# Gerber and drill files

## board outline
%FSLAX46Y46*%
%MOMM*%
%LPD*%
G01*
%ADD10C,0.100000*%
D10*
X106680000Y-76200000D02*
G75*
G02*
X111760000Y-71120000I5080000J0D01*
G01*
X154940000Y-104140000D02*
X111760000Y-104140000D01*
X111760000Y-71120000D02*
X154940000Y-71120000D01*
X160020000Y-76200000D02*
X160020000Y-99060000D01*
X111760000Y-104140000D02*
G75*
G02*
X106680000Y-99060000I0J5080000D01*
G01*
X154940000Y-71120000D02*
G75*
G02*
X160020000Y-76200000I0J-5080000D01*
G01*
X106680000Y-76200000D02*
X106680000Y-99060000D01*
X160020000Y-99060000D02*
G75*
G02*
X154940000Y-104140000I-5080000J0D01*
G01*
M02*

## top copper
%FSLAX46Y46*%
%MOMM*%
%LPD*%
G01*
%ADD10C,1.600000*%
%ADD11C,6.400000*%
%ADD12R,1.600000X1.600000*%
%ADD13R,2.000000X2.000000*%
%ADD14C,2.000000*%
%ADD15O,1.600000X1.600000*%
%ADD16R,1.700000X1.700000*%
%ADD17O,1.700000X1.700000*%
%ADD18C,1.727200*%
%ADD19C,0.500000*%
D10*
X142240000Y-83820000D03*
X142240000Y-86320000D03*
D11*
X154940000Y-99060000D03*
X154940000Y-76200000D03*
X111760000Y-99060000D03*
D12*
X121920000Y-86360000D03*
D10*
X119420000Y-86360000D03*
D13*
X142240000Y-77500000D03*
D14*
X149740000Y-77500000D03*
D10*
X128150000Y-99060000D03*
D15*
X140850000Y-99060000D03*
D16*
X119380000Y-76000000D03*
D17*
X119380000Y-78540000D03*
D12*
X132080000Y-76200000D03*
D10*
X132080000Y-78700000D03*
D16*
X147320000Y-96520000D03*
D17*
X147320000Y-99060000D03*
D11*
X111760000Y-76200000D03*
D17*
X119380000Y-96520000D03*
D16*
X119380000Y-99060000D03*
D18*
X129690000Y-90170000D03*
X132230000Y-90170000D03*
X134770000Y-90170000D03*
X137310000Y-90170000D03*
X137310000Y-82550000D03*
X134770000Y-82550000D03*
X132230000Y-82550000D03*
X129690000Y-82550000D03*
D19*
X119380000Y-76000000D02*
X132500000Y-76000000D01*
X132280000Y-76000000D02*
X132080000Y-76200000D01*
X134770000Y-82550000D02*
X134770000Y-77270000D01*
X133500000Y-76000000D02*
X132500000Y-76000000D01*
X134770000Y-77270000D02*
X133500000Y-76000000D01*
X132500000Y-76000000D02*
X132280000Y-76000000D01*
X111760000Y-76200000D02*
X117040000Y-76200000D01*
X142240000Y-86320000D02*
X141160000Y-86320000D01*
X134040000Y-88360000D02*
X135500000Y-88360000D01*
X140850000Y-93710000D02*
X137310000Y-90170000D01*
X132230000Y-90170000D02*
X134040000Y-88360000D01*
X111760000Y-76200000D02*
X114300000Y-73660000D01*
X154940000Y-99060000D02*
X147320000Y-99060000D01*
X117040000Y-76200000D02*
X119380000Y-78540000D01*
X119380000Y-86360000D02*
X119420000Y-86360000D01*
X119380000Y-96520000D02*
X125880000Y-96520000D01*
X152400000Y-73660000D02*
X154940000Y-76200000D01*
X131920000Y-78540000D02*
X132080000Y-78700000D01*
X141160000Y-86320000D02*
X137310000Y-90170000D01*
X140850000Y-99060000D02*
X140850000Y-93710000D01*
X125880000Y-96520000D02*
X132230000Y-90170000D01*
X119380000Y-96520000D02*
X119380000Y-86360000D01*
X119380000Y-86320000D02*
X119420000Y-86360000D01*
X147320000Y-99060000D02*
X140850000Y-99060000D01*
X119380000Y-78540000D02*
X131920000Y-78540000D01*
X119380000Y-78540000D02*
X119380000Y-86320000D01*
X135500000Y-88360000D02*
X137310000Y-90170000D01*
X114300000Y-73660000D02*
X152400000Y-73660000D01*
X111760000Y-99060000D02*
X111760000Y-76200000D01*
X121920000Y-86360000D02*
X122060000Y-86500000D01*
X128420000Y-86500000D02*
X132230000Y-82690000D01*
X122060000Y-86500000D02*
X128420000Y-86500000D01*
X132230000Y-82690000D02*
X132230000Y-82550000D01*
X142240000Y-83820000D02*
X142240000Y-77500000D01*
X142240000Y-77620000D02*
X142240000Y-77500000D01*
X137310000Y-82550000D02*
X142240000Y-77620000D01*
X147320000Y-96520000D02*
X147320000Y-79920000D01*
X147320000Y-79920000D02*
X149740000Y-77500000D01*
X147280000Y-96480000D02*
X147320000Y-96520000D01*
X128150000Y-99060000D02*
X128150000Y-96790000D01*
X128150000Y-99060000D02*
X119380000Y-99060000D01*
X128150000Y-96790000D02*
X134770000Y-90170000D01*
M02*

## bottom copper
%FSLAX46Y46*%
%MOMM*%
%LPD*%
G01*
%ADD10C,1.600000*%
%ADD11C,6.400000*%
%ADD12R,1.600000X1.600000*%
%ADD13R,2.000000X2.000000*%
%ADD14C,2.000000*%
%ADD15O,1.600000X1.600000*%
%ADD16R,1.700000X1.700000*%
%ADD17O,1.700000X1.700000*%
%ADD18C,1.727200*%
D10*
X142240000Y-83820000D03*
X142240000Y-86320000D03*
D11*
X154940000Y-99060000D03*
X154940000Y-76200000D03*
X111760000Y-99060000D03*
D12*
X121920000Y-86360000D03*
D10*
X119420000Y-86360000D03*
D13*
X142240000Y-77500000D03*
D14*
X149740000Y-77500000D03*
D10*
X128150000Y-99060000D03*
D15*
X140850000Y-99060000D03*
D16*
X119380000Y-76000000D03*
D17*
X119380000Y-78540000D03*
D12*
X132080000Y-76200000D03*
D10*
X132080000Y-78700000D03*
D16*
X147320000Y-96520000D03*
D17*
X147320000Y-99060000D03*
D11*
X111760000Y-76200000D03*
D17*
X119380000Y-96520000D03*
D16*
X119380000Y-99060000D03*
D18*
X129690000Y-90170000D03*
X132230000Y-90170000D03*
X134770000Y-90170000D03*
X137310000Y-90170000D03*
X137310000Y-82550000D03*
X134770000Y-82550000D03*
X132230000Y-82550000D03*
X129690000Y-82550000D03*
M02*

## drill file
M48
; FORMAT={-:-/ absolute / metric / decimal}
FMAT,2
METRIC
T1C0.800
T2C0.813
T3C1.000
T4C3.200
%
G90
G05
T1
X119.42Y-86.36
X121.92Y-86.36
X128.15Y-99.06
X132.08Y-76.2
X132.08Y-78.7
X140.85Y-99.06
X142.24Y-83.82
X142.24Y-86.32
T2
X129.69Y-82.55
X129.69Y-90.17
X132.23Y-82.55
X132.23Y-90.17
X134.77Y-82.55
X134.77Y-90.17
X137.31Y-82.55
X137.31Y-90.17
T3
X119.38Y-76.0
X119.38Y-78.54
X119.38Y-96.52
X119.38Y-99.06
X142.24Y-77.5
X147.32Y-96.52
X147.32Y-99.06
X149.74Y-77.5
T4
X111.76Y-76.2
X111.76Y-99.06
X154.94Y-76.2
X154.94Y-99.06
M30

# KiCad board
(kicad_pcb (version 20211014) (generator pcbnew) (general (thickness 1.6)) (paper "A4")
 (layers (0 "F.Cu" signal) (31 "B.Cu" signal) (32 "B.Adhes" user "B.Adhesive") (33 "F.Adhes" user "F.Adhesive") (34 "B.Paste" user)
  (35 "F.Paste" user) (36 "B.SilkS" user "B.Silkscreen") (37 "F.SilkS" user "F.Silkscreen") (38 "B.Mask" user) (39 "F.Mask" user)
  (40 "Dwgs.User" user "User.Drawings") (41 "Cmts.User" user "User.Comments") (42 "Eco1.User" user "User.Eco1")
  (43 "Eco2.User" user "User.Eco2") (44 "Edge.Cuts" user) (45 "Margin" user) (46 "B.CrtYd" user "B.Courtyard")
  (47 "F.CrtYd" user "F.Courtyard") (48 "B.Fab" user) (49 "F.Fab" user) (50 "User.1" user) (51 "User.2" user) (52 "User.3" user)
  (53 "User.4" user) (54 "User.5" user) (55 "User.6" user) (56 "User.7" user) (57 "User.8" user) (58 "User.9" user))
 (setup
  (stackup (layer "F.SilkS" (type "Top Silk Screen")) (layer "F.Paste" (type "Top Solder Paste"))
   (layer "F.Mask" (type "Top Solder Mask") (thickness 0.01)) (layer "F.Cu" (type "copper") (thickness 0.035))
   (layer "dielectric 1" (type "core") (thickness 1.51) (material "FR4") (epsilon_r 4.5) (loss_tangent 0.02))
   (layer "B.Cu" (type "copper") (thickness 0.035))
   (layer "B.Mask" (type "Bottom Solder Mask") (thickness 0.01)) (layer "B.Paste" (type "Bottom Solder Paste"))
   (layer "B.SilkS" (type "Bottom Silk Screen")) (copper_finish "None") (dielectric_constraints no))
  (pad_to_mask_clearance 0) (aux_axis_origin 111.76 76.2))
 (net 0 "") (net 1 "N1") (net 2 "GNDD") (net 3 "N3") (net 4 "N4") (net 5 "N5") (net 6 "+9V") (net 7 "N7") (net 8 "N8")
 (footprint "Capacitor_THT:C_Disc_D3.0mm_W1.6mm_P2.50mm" (layer "F.Cu") (at 142.24 83.82 -90)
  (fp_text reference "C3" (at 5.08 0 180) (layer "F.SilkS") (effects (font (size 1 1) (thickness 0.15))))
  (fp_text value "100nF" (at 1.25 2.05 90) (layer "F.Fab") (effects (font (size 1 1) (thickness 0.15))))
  (pad "1" thru_hole circle (at 0 0 270) (size 1.6 1.6) (drill 0.8) (layers *.Cu *.Mask) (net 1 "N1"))
  (pad "2" thru_hole circle (at 2.5 0 270) (size 1.6 1.6) (drill 0.8) (layers *.Cu *.Mask) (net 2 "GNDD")))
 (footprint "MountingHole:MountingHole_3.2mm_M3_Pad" (layer "F.Cu") (at 154.94 99.06)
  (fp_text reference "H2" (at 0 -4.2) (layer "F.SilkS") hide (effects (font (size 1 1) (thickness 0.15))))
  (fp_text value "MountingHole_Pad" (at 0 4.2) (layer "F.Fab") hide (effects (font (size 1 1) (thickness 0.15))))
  (pad "1" thru_hole circle (at 0 0) (size 6.4 6.4) (drill 3.2) (layers *.Cu *.Mask) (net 2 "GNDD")))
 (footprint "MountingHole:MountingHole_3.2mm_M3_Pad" (layer "F.Cu") (at 154.94 76.2)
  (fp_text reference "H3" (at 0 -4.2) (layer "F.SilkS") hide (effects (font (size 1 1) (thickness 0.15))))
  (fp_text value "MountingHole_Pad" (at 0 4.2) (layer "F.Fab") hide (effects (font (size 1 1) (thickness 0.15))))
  (pad "1" thru_hole circle (at 0 0) (size 6.4 6.4) (drill 3.2) (layers *.Cu *.Mask) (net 2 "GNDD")))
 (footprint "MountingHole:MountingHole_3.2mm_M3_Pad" (layer "F.Cu") (at 111.76 99.06)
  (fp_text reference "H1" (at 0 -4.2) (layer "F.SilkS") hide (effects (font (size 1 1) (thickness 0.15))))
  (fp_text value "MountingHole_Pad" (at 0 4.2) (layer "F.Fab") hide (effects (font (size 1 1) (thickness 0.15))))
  (pad "1" thru_hole circle (at 0 0) (size 6.4 6.4) (drill 3.2) (layers *.Cu *.Mask) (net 2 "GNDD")))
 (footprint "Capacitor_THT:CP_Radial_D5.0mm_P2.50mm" (layer "F.Cu") (at 121.92 86.36 180)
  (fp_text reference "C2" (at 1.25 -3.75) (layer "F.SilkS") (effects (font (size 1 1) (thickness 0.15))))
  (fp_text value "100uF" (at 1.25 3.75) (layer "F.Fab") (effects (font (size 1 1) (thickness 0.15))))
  (pad "1" thru_hole rect (at 0 0 180) (size 1.6 1.6) (drill 0.8) (layers *.Cu *.Mask) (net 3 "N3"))
  (pad "2" thru_hole circle (at 2.5 0 180) (size 1.6 1.6) (drill 0.8) (layers *.Cu *.Mask) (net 2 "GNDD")))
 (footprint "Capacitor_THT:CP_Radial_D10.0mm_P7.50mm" (layer "F.Cu") (at 142.24 77.5)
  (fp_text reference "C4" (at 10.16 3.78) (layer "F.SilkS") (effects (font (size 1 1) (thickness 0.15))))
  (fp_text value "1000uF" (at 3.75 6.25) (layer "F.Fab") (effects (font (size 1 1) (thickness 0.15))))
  (pad "1" thru_hole rect (at 0 0) (size 2 2) (drill 1) (layers *.Cu *.Mask) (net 1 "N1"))
  (pad "2" thru_hole circle (at 7.5 0) (size 2 2) (drill 1) (layers *.Cu *.Mask) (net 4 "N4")))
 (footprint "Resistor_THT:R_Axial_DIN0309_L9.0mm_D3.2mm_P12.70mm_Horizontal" (layer "F.Cu") (at 128.15 99.06)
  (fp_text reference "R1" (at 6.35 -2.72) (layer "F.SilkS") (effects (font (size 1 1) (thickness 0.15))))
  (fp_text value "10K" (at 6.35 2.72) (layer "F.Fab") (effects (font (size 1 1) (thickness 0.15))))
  (pad "1" thru_hole circle (at 0 0) (size 1.6 1.6) (drill 0.8) (layers *.Cu *.Mask) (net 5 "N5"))
  (pad "2" thru_hole oval (at 12.7 0) (size 1.6 1.6) (drill 0.8) (layers *.Cu *.Mask) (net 2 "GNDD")))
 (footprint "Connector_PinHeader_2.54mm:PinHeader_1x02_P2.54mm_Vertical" (layer "F.Cu") (at 119.38 76)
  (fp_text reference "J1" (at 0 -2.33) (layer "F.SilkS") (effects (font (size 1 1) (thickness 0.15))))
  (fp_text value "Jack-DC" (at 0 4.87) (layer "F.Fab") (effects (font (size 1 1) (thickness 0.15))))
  (pad "1" thru_hole rect (at 0 0) (size 1.7 1.7) (drill 1) (layers *.Cu *.Mask) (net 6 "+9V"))
  (pad "2" thru_hole oval (at 0 2.54) (size 1.7 1.7) (drill 1) (layers *.Cu *.Mask) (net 2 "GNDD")))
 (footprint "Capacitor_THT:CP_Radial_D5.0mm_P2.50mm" (layer "F.Cu") (at 132.08 76.2 -90)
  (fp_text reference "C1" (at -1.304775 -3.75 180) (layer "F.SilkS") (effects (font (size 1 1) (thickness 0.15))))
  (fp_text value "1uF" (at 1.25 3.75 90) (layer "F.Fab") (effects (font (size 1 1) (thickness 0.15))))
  (pad "1" thru_hole rect (at 0 0 270) (size 1.6 1.6) (drill 0.8) (layers *.Cu *.Mask) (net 6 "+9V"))
  (pad "2" thru_hole circle (at 2.5 0 270) (size 1.6 1.6) (drill 0.8) (layers *.Cu *.Mask) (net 2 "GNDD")))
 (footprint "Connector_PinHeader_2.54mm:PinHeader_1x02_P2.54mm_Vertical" (layer "F.Cu") (at 147.32 96.52)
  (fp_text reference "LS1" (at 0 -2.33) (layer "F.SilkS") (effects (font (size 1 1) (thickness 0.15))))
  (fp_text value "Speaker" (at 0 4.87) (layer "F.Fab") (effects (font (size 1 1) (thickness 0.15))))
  (pad "1" thru_hole rect (at 0 0) (size 1.7 1.7) (drill 1) (layers *.Cu *.Mask) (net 4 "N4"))
  (pad "2" thru_hole oval (at 0 2.54) (size 1.7 1.7) (drill 1) (layers *.Cu *.Mask) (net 2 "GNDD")))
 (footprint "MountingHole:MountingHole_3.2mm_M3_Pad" (layer "F.Cu") (at 111.76 76.2)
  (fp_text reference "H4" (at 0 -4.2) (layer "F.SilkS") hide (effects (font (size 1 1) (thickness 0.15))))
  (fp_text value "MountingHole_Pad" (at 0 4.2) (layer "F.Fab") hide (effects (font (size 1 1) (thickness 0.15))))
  (pad "1" thru_hole circle (at 0 0) (size 6.4 6.4) (drill 3.2) (layers *.Cu *.Mask) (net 2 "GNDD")))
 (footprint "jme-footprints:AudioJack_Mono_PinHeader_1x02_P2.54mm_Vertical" (layer "F.Cu") (at 119.38 99.06 180)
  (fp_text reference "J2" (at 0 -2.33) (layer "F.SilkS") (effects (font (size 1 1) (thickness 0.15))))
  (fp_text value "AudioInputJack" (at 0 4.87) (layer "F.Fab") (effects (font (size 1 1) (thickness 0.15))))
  (pad "S" thru_hole oval (at 0 2.54 180) (size 1.7 1.7) (drill 1) (layers *.Cu *.Mask) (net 2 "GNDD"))
  (pad "T" thru_hole rect (at 0 0 180) (size 1.7 1.7) (drill 1) (layers *.Cu *.Mask) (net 5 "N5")))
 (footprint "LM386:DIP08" (layer "F.Cu") (at 133.5 86.36)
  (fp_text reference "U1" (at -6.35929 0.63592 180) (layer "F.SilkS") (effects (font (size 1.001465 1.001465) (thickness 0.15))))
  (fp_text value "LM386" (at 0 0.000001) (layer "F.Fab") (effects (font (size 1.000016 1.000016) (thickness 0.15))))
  (pad "1" thru_hole circle locked (at -3.81 3.81) (size 1.7272 1.7272) (drill 0.8128) (layers *.Cu *.Mask) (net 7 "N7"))
  (pad "2" thru_hole circle locked (at -1.27 3.81) (size 1.7272 1.7272) (drill 0.8128) (layers *.Cu *.Mask) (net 2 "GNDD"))
  (pad "3" thru_hole circle locked (at 1.27 3.81) (size 1.7272 1.7272) (drill 0.8128) (layers *.Cu *.Mask) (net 5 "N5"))
  (pad "4" thru_hole circle locked (at 3.81 3.81) (size 1.7272 1.7272) (drill 0.8128) (layers *.Cu *.Mask) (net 2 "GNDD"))
  (pad "5" thru_hole circle locked (at 3.81 -3.81) (size 1.7272 1.7272) (drill 0.8128) (layers *.Cu *.Mask) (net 1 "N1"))
  (pad "6" thru_hole circle locked (at 1.27 -3.81) (size 1.7272 1.7272) (drill 0.8128) (layers *.Cu *.Mask) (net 6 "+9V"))
  (pad "7" thru_hole circle locked (at -1.27 -3.81) (size 1.7272 1.7272) (drill 0.8128) (layers *.Cu *.Mask) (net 3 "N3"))
  (pad "8" thru_hole circle locked (at -3.81 -3.81) (size 1.7272 1.7272) (drill 0.8128) (layers *.Cu *.Mask) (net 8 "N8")))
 (gr_arc (start 106.68 76.2) (mid 108.167898 72.607898) (end 111.76 71.12) (layer "Edge.Cuts") (width 0.1))
 (gr_line (start 154.94 104.14) (end 111.76 104.14) (layer "Edge.Cuts") (width 0.1))
 (gr_line (start 111.76 71.12) (end 154.94 71.12) (layer "Edge.Cuts") (width 0.1))
 (gr_line (start 160.02 76.2) (end 160.02 99.06) (layer "Edge.Cuts") (width 0.1))
 (gr_arc (start 111.76 104.14) (mid 108.167898 102.652102) (end 106.68 99.06) (layer "Edge.Cuts") (width 0.1))
 (gr_arc (start 154.94 71.12) (mid 158.532102 72.607898) (end 160.02 76.2) (layer "Edge.Cuts") (width 0.1))
 (gr_line (start 106.68 76.2) (end 106.68 99.06) (layer "Edge.Cuts") (width 0.1))
 (gr_arc (start 160.02 99.06) (mid 158.532102 102.652102) (end 154.94 104.14) (layer "Edge.Cuts") (width 0.1))
 (segment (start 119.38 76) (end 132.5 76) (width 0.5) (layer "F.Cu") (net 6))
 (segment (start 132.28 76) (end 132.08 76.2) (width 0.5) (layer "F.Cu") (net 6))
 (segment (start 134.77 82.55) (end 134.77 77.27) (width 0.5) (layer "F.Cu") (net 6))
 (segment (start 133.5 76) (end 132.5 76) (width 0.5) (layer "F.Cu") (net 6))
 (segment (start 134.77 77.27) (end 133.5 76) (width 0.5) (layer "F.Cu") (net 6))
 (segment (start 132.5 76) (end 132.28 76) (width 0.5) (layer "F.Cu") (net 6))
 (segment (start 111.76 76.2) (end 117.04 76.2) (width 0.5) (layer "F.Cu") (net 2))
 (segment (start 142.24 86.32) (end 141.16 86.32) (width 0.5) (layer "F.Cu") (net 2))
 (segment (start 134.04 88.36) (end 135.5 88.36) (width 0.5) (layer "F.Cu") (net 2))
 (segment (start 140.85 93.71) (end 137.31 90.17) (width 0.5) (layer "F.Cu") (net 2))
 (segment (start 132.23 90.17) (end 134.04 88.36) (width 0.5) (layer "F.Cu") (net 2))
 (segment (start 111.76 76.2) (end 114.3 73.66) (width 0.5) (layer "F.Cu") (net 2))
 (segment (start 154.94 99.06) (end 147.32 99.06) (width 0.5) (layer "F.Cu") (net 2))
 (segment (start 117.04 76.2) (end 119.38 78.54) (width 0.5) (layer "F.Cu") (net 2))
 (segment (start 119.38 86.36) (end 119.42 86.36) (width 0.5) (layer "F.Cu") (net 2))
 (segment (start 119.38 96.52) (end 125.88 96.52) (width 0.5) (layer "F.Cu") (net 2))
 (segment (start 152.4 73.66) (end 154.94 76.2) (width 0.5) (layer "F.Cu") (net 2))
 (segment (start 131.92 78.54) (end 132.08 78.7) (width 0.5) (layer "F.Cu") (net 2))
 (segment (start 141.16 86.32) (end 137.31 90.17) (width 0.5) (layer "F.Cu") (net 2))
 (segment (start 140.85 99.06) (end 140.85 93.71) (width 0.5) (layer "F.Cu") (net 2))
 (segment (start 125.88 96.52) (end 132.23 90.17) (width 0.5) (layer "F.Cu") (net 2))
 (segment (start 119.38 96.52) (end 119.38 86.36) (width 0.5) (layer "F.Cu") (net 2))
 (segment (start 119.38 86.32) (end 119.42 86.36) (width 0.5) (layer "F.Cu") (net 2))
 (segment (start 147.32 99.06) (end 140.85 99.06) (width 0.5) (layer "F.Cu") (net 2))
 (segment (start 119.38 78.54) (end 131.92 78.54) (width 0.5) (layer "F.Cu") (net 2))
 (segment (start 119.38 78.54) (end 119.38 86.32) (width 0.5) (layer "F.Cu") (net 2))
 (segment (start 135.5 88.36) (end 137.31 90.17) (width 0.5) (layer "F.Cu") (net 2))
 (segment (start 114.3 73.66) (end 152.4 73.66) (width 0.5) (layer "F.Cu") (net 2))
 (segment (start 111.76 99.06) (end 111.76 76.2) (width 0.5) (layer "F.Cu") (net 2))
 (segment (start 121.92 86.36) (end 122.06 86.5) (width 0.5) (layer "F.Cu") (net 3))
 (segment (start 128.42 86.5) (end 132.23 82.69) (width 0.5) (layer "F.Cu") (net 3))
 (segment (start 122.06 86.5) (end 128.42 86.5) (width 0.5) (layer "F.Cu") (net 3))
 (segment (start 132.23 82.69) (end 132.23 82.55) (width 0.5) (layer "F.Cu") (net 3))
 (segment (start 142.24 83.82) (end 142.24 77.5) (width 0.5) (layer "F.Cu") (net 1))
 (segment (start 142.24 77.62) (end 142.24 77.5) (width 0.5) (layer "F.Cu") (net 1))
 (segment (start 137.31 82.55) (end 142.24 77.62) (width 0.5) (layer "F.Cu") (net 1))
 (segment (start 147.32 96.52) (end 147.32 79.92) (width 0.5) (layer "F.Cu") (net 4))
 (segment (start 147.32 79.92) (end 149.74 77.5) (width 0.5) (layer "F.Cu") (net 4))
 (segment (start 147.28 96.48) (end 147.32 96.52) (width 0.5) (layer "F.Cu") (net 4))
 (segment (start 128.15 99.06) (end 128.15 96.79) (width 0.5) (layer "F.Cu") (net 5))
 (segment (start 128.15 99.06) (end 119.38 99.06) (width 0.5) (layer "F.Cu") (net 5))
 (segment (start 128.15 96.79) (end 134.77 90.17) (width 0.5) (layer "F.Cu") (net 5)))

